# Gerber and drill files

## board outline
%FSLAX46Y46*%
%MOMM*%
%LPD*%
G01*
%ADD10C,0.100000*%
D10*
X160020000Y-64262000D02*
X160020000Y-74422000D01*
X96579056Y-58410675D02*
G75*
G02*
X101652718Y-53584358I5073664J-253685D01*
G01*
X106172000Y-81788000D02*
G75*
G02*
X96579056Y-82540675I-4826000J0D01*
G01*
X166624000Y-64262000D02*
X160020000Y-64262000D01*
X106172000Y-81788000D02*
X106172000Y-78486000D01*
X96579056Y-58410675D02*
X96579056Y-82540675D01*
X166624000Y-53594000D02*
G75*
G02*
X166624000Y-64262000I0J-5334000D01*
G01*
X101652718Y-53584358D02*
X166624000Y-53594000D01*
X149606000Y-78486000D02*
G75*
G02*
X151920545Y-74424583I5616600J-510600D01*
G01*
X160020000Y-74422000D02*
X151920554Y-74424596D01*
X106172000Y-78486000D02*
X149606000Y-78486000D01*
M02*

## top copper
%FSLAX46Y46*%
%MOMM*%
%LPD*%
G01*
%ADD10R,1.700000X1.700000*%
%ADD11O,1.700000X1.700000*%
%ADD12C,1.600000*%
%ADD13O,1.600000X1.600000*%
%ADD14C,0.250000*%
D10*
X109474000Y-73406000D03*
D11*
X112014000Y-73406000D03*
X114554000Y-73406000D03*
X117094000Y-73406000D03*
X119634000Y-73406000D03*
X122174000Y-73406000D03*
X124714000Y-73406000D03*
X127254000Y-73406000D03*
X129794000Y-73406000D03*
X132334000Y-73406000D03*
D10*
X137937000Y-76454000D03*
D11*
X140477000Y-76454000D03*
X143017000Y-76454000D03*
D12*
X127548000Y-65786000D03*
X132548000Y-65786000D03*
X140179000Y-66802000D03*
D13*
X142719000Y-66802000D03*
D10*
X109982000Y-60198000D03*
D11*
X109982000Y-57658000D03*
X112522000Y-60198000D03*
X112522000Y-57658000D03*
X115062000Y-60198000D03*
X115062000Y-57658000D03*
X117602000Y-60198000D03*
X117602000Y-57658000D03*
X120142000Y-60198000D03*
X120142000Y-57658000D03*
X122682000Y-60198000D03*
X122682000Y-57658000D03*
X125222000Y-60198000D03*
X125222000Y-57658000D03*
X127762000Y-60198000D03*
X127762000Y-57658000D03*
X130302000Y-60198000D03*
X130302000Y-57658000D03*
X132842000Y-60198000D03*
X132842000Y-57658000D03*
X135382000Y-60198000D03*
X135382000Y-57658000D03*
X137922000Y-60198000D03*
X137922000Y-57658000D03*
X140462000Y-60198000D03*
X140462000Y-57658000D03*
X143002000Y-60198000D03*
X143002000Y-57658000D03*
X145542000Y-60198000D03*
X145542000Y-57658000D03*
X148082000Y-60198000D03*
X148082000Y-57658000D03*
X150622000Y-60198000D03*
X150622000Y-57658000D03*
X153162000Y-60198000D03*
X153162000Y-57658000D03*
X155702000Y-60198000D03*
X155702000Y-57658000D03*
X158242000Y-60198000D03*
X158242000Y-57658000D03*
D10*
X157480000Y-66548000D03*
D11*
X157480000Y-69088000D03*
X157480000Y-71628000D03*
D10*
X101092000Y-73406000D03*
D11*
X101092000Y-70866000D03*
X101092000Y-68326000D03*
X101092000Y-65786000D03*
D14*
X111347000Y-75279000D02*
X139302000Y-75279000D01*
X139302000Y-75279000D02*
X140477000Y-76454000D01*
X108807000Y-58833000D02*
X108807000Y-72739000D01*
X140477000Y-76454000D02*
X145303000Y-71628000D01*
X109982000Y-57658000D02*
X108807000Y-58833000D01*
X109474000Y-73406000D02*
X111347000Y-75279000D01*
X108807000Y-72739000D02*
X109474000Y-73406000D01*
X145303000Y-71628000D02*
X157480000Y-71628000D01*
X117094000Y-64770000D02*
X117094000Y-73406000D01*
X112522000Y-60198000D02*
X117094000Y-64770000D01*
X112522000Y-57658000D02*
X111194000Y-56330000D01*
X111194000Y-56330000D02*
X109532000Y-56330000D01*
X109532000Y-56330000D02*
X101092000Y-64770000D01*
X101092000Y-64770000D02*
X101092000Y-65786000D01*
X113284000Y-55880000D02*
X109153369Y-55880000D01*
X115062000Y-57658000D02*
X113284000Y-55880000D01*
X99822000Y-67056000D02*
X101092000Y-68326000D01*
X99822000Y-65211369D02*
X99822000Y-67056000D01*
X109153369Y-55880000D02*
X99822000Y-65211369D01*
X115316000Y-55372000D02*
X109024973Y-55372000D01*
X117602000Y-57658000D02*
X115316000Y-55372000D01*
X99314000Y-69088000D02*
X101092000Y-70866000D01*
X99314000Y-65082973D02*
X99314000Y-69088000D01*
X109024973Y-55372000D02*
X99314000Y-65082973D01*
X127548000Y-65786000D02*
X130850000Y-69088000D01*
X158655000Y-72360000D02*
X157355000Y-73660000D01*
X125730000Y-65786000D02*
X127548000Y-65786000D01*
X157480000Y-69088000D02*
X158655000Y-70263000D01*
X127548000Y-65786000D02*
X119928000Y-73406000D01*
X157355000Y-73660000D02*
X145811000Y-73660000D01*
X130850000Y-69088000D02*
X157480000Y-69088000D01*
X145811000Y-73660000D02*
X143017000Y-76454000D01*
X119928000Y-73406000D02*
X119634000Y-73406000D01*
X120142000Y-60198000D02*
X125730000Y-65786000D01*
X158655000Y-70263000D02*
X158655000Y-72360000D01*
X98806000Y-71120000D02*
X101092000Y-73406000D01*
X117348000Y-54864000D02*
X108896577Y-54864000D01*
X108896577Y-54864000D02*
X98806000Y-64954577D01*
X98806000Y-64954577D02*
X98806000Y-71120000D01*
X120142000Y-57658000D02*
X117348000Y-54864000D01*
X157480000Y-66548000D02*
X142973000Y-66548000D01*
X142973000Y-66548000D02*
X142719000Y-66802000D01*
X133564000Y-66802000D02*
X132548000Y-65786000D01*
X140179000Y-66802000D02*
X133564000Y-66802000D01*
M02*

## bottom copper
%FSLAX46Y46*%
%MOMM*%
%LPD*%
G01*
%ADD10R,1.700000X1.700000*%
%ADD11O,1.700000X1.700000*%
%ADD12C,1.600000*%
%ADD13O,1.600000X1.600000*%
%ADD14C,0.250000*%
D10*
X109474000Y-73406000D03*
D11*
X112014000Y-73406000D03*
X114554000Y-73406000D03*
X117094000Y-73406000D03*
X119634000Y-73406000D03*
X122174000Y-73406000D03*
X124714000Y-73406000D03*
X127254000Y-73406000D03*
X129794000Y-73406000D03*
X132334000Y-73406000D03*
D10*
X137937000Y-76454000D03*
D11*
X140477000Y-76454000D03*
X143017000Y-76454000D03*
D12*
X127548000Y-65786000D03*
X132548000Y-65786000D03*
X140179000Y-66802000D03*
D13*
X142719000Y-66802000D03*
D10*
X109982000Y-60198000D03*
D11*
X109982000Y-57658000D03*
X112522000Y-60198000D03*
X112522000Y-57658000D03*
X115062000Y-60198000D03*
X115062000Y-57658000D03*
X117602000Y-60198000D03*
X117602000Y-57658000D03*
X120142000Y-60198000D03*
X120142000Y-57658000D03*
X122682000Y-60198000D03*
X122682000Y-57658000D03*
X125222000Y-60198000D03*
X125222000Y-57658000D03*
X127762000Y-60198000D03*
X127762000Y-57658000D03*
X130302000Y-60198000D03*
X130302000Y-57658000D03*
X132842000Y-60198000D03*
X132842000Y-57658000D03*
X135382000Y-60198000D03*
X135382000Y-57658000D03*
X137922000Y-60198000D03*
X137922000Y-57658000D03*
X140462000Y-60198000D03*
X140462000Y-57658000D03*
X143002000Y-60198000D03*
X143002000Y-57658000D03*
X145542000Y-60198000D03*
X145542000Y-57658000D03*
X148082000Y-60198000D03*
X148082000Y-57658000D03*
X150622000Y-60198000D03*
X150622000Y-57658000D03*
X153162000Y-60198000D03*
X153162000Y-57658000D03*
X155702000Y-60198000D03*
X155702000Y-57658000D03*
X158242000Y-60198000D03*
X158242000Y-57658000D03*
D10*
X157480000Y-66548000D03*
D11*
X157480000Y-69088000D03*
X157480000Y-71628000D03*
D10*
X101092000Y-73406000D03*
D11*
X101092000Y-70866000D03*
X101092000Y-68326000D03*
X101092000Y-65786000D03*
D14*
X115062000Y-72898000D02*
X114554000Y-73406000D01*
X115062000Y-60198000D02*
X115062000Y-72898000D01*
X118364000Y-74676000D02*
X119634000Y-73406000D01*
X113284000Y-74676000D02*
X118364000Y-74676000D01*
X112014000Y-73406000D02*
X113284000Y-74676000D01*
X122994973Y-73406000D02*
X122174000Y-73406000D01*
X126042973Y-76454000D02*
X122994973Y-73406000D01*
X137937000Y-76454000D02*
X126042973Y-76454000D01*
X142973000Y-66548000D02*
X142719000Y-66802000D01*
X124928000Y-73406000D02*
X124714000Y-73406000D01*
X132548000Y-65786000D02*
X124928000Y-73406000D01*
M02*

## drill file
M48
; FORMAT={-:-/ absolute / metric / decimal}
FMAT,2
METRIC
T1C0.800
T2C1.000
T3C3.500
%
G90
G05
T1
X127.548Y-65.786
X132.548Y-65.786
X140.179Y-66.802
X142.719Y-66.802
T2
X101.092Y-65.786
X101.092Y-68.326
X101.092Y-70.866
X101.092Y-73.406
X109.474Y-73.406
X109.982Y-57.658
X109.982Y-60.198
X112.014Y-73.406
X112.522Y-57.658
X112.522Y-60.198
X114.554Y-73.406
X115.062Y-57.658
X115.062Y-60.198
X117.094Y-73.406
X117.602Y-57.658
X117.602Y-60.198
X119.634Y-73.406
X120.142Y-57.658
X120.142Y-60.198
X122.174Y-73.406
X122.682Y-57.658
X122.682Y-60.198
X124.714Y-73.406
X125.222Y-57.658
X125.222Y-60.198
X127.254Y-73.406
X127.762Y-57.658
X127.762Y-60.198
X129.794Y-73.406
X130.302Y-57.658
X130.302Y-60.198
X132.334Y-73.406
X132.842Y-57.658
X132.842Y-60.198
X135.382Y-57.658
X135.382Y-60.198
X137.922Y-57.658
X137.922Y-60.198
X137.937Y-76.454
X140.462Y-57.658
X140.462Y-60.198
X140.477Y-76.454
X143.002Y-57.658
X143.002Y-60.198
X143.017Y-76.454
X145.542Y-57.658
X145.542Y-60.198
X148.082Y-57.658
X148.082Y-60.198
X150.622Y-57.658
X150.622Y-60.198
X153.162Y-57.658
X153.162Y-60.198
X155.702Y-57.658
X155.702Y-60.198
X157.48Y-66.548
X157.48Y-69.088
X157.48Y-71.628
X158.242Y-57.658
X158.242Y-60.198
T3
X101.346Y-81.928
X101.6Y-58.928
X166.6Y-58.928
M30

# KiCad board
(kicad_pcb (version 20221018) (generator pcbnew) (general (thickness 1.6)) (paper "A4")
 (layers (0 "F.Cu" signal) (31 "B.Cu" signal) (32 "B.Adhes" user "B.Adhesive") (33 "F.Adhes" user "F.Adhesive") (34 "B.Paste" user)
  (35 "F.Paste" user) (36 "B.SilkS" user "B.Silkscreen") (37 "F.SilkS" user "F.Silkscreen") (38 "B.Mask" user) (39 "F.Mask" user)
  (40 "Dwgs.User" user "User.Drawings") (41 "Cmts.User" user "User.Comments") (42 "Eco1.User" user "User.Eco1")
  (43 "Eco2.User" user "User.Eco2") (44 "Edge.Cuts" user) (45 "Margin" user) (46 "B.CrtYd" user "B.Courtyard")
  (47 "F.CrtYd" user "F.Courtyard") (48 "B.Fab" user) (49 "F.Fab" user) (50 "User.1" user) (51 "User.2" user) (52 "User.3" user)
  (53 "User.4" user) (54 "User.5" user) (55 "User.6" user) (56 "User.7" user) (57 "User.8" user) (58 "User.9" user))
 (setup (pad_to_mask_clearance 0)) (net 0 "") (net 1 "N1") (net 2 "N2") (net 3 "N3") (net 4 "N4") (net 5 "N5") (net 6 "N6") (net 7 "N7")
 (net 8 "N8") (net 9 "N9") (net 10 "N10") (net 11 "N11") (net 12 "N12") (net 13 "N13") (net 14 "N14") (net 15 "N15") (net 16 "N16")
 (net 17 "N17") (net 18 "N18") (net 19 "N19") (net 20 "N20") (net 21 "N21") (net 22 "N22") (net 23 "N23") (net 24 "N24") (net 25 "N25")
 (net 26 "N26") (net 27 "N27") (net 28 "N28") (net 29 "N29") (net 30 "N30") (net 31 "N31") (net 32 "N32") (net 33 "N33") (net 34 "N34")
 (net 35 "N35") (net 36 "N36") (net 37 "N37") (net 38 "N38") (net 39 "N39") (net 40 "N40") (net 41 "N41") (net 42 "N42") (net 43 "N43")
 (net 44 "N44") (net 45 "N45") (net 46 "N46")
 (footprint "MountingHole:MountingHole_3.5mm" (layer "F.Cu") (at 166.6 58.928)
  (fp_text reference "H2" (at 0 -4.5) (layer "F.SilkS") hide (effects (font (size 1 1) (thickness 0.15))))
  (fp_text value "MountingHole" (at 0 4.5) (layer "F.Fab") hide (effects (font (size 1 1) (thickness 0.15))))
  (pad "" np_thru_hole circle (at 0 0) (size 3.5 3.5) (drill 3.5) (layers "*.Cu" "*.Mask")))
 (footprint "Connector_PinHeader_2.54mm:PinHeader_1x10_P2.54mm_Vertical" (layer "F.Cu") (at 109.474 73.406 90)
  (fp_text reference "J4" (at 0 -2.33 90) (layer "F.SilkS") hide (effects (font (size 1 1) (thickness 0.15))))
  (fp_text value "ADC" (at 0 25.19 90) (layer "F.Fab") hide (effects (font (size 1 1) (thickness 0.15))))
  (pad "1" thru_hole rect (at 0 0 90) (size 1.7 1.7) (drill 1) (layers "*.Cu" "*.Mask") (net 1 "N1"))
  (pad "2" thru_hole oval (at 0 2.54 90) (size 1.7 1.7) (drill 1) (layers "*.Cu" "*.Mask") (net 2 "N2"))
  (pad "3" thru_hole oval (at 0 5.08 90) (size 1.7 1.7) (drill 1) (layers "*.Cu" "*.Mask") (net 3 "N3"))
  (pad "4" thru_hole oval (at 0 7.62 90) (size 1.7 1.7) (drill 1) (layers "*.Cu" "*.Mask") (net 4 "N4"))
  (pad "5" thru_hole oval (at 0 10.16 90) (size 1.7 1.7) (drill 1) (layers "*.Cu" "*.Mask") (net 2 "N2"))
  (pad "6" thru_hole oval (at 0 12.7 90) (size 1.7 1.7) (drill 1) (layers "*.Cu" "*.Mask") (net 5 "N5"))
  (pad "7" thru_hole oval (at 0 15.24 90) (size 1.7 1.7) (drill 1) (layers "*.Cu" "*.Mask") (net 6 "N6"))
  (pad "8" thru_hole oval (at 0 17.78 90) (size 1.7 1.7) (drill 1) (layers "*.Cu" "*.Mask") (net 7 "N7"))
  (pad "9" thru_hole oval (at 0 20.32 90) (size 1.7 1.7) (drill 1) (layers "*.Cu" "*.Mask") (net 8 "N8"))
  (pad "10" thru_hole oval (at 0 22.86 90) (size 1.7 1.7) (drill 1) (layers "*.Cu" "*.Mask") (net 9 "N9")))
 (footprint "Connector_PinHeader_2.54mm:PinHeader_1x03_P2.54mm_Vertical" (layer "F.Cu") (at 137.937 76.454 90)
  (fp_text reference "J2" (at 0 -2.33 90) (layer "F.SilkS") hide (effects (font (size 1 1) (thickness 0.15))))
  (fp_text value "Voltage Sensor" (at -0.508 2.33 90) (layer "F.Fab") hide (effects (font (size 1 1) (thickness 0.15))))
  (pad "1" thru_hole rect (at 0 0 90) (size 1.7 1.7) (drill 1) (layers "*.Cu" "*.Mask") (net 5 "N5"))
  (pad "2" thru_hole oval (at 0 2.54 90) (size 1.7 1.7) (drill 1) (layers "*.Cu" "*.Mask") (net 1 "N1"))
  (pad "3" thru_hole oval (at 0 5.08 90) (size 1.7 1.7) (drill 1) (layers "*.Cu" "*.Mask") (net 2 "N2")))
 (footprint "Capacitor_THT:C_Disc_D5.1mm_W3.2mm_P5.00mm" (layer "F.Cu") (at 127.548 65.786)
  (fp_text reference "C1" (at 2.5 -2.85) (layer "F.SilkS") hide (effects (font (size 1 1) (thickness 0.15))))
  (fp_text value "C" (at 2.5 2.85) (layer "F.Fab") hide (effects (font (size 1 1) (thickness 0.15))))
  (pad "1" thru_hole circle (at 0 0) (size 1.6 1.6) (drill 0.8) (layers "*.Cu" "*.Mask") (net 2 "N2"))
  (pad "2" thru_hole circle (at 5 0) (size 1.6 1.6) (drill 0.8) (layers "*.Cu" "*.Mask") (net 6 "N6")))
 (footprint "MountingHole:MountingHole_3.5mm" (layer "F.Cu") (at 101.346 81.928)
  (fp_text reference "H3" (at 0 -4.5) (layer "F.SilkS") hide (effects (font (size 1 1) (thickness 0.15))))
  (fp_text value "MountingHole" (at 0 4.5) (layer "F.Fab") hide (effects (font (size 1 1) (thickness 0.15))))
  (pad "" np_thru_hole circle (at 0 0) (size 3.5 3.5) (drill 3.5) (layers "*.Cu" "*.Mask")))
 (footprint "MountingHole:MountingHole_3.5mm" (layer "F.Cu") (at 101.6 58.928)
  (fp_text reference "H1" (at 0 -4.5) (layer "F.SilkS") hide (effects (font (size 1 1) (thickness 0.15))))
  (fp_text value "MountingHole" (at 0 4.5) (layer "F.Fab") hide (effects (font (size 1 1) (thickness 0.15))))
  (pad "" np_thru_hole circle (at 0 0) (size 3.5 3.5) (drill 3.5) (layers "*.Cu" "*.Mask")))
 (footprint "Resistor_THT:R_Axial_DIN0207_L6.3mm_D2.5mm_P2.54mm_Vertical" (layer "F.Cu") (at 140.179 66.802)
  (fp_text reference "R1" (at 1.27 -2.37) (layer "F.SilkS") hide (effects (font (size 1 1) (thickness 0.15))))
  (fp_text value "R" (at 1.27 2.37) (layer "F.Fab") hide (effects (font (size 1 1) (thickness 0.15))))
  (pad "1" thru_hole circle (at 0 0) (size 1.6 1.6) (drill 0.8) (layers "*.Cu" "*.Mask") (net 6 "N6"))
  (pad "2" thru_hole oval (at 2.54 0) (size 1.6 1.6) (drill 0.8) (layers "*.Cu" "*.Mask") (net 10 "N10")))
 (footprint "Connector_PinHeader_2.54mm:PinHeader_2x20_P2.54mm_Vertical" (layer "F.Cu") (at 109.982 60.198 90)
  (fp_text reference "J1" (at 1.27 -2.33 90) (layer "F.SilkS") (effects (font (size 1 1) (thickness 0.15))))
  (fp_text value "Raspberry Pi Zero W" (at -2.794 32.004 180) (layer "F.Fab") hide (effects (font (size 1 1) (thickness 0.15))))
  (pad "1" thru_hole rect (at 0 0 90) (size 1.7 1.7) (drill 1) (layers "*.Cu" "*.Mask") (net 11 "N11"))
  (pad "2" thru_hole oval (at 2.54 0 90) (size 1.7 1.7) (drill 1) (layers "*.Cu" "*.Mask") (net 1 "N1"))
  (pad "3" thru_hole oval (at 0 2.54 90) (size 1.7 1.7) (drill 1) (layers "*.Cu" "*.Mask") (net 4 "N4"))
  (pad "4" thru_hole oval (at 2.54 2.54 90) (size 1.7 1.7) (drill 1) (layers "*.Cu" "*.Mask") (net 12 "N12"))
  (pad "5" thru_hole oval (at 0 5.08 90) (size 1.7 1.7) (drill 1) (layers "*.Cu" "*.Mask") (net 3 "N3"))
  (pad "6" thru_hole oval (at 2.54 5.08 90) (size 1.7 1.7) (drill 1) (layers "*.Cu" "*.Mask") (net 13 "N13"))
  (pad "7" thru_hole oval (at 0 7.62 90) (size 1.7 1.7) (drill 1) (layers "*.Cu" "*.Mask") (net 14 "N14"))
  (pad "8" thru_hole oval (at 2.54 7.62 90) (size 1.7 1.7) (drill 1) (layers "*.Cu" "*.Mask") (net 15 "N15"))
  (pad "9" thru_hole oval (at 0 10.16 90) (size 1.7 1.7) (drill 1) (layers "*.Cu" "*.Mask") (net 2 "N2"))
  (pad "10" thru_hole oval (at 2.54 10.16 90) (size 1.7 1.7) (drill 1) (layers "*.Cu" "*.Mask") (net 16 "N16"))
  (pad "11" thru_hole oval (at 0 12.7 90) (size 1.7 1.7) (drill 1) (layers "*.Cu" "*.Mask") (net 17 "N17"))
  (pad "12" thru_hole oval (at 2.54 12.7 90) (size 1.7 1.7) (drill 1) (layers "*.Cu" "*.Mask") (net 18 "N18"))
  (pad "13" thru_hole oval (at 0 15.24 90) (size 1.7 1.7) (drill 1) (layers "*.Cu" "*.Mask") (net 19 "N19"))
  (pad "14" thru_hole oval (at 2.54 15.24 90) (size 1.7 1.7) (drill 1) (layers "*.Cu" "*.Mask") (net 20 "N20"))
  (pad "15" thru_hole oval (at 0 17.78 90) (size 1.7 1.7) (drill 1) (layers "*.Cu" "*.Mask") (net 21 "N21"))
  (pad "16" thru_hole oval (at 2.54 17.78 90) (size 1.7 1.7) (drill 1) (layers "*.Cu" "*.Mask") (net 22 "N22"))
  (pad "17" thru_hole oval (at 0 20.32 90) (size 1.7 1.7) (drill 1) (layers "*.Cu" "*.Mask") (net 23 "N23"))
  (pad "18" thru_hole oval (at 2.54 20.32 90) (size 1.7 1.7) (drill 1) (layers "*.Cu" "*.Mask") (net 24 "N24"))
  (pad "19" thru_hole oval (at 0 22.86 90) (size 1.7 1.7) (drill 1) (layers "*.Cu" "*.Mask") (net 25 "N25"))
  (pad "20" thru_hole oval (at 2.54 22.86 90) (size 1.7 1.7) (drill 1) (layers "*.Cu" "*.Mask") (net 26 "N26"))
  (pad "21" thru_hole oval (at 0 25.4 90) (size 1.7 1.7) (drill 1) (layers "*.Cu" "*.Mask") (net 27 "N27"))
  (pad "22" thru_hole oval (at 2.54 25.4 90) (size 1.7 1.7) (drill 1) (layers "*.Cu" "*.Mask") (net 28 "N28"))
  (pad "23" thru_hole oval (at 0 27.94 90) (size 1.7 1.7) (drill 1) (layers "*.Cu" "*.Mask") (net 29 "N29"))
  (pad "24" thru_hole oval (at 2.54 27.94 90) (size 1.7 1.7) (drill 1) (layers "*.Cu" "*.Mask") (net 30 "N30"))
  (pad "25" thru_hole oval (at 0 30.48 90) (size 1.7 1.7) (drill 1) (layers "*.Cu" "*.Mask") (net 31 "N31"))
  (pad "26" thru_hole oval (at 2.54 30.48 90) (size 1.7 1.7) (drill 1) (layers "*.Cu" "*.Mask") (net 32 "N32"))
  (pad "27" thru_hole oval (at 0 33.02 90) (size 1.7 1.7) (drill 1) (layers "*.Cu" "*.Mask") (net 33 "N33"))
  (pad "28" thru_hole oval (at 2.54 33.02 90) (size 1.7 1.7) (drill 1) (layers "*.Cu" "*.Mask") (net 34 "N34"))
  (pad "29" thru_hole oval (at 0 35.56 90) (size 1.7 1.7) (drill 1) (layers "*.Cu" "*.Mask") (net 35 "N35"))
  (pad "30" thru_hole oval (at 2.54 35.56 90) (size 1.7 1.7) (drill 1) (layers "*.Cu" "*.Mask") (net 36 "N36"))
  (pad "31" thru_hole oval (at 0 38.1 90) (size 1.7 1.7) (drill 1) (layers "*.Cu" "*.Mask") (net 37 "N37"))
  (pad "32" thru_hole oval (at 2.54 38.1 90) (size 1.7 1.7) (drill 1) (layers "*.Cu" "*.Mask") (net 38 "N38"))
  (pad "33" thru_hole oval (at 0 40.64 90) (size 1.7 1.7) (drill 1) (layers "*.Cu" "*.Mask") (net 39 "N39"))
  (pad "34" thru_hole oval (at 2.54 40.64 90) (size 1.7 1.7) (drill 1) (layers "*.Cu" "*.Mask") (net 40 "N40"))
  (pad "35" thru_hole oval (at 0 43.18 90) (size 1.7 1.7) (drill 1) (layers "*.Cu" "*.Mask") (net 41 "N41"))
  (pad "36" thru_hole oval (at 2.54 43.18 90) (size 1.7 1.7) (drill 1) (layers "*.Cu" "*.Mask") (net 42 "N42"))
  (pad "37" thru_hole oval (at 0 45.72 90) (size 1.7 1.7) (drill 1) (layers "*.Cu" "*.Mask") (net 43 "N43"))
  (pad "38" thru_hole oval (at 2.54 45.72 90) (size 1.7 1.7) (drill 1) (layers "*.Cu" "*.Mask") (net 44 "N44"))
  (pad "39" thru_hole oval (at 0 48.26 90) (size 1.7 1.7) (drill 1) (layers "*.Cu" "*.Mask") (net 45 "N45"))
  (pad "40" thru_hole oval (at 2.54 48.26 90) (size 1.7 1.7) (drill 1) (layers "*.Cu" "*.Mask") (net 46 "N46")))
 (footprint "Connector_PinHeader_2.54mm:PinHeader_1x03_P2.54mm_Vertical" (layer "F.Cu") (at 157.48 66.548)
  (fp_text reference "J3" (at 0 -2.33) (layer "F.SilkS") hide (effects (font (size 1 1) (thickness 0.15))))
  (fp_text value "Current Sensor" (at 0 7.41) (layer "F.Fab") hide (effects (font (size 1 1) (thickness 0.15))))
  (pad "1" thru_hole rect (at 0 0) (size 1.7 1.7) (drill 1) (layers "*.Cu" "*.Mask") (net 10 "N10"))
  (pad "2" thru_hole oval (at 0 2.54) (size 1.7 1.7) (drill 1) (layers "*.Cu" "*.Mask") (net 2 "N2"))
  (pad "3" thru_hole oval (at 0 5.08) (size 1.7 1.7) (drill 1) (layers "*.Cu" "*.Mask") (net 1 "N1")))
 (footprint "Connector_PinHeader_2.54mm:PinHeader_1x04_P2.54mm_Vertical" (layer "F.Cu") (at 101.092 73.406 180)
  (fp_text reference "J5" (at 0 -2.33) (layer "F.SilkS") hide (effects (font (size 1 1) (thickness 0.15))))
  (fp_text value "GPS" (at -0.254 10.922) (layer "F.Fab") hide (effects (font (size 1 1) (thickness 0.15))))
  (pad "1" thru_hole rect (at 0 0 180) (size 1.7 1.7) (drill 1) (layers "*.Cu" "*.Mask") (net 16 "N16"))
  (pad "2" thru_hole oval (at 0 2.54 180) (size 1.7 1.7) (drill 1) (layers "*.Cu" "*.Mask") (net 15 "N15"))
  (pad "3" thru_hole oval (at 0 5.08 180) (size 1.7 1.7) (drill 1) (layers "*.Cu" "*.Mask") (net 13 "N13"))
  (pad "4" thru_hole oval (at 0 7.62 180) (size 1.7 1.7) (drill 1) (layers "*.Cu" "*.Mask") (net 12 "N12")))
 (gr_line (start 160.02 64.262) (end 160.02 74.422) (stroke (width 0.1) (type default)) (layer "Edge.Cuts"))
 (gr_arc (start 96.579056 58.410675) (mid 98.151455 54.983658) (end 101.652718 53.584358) (stroke (width 0.1) (type default))
  (layer "Edge.Cuts"))
 (gr_arc (start 106.172 81.788) (mid 101.723494 86.599213) (end 96.579056 82.540675) (stroke (width 0.1) (type default)) (layer "Edge.Cuts"))
 (gr_line (start 166.624 64.262) (end 160.02 64.262) (stroke (width 0.1) (type default)) (layer "Edge.Cuts"))
 (gr_line (start 106.172 81.788) (end 106.172 78.486) (stroke (width 0.1) (type default)) (layer "Edge.Cuts"))
 (gr_line (start 96.579056 58.410675) (end 96.579056 82.540675) (stroke (width 0.1) (type default)) (layer "Edge.Cuts"))
 (gr_arc (start 166.624 53.594) (mid 171.958 58.928) (end 166.624 64.262) (stroke (width 0.1) (type default)) (layer "Edge.Cuts"))
 (gr_line (start 101.652718 53.584358) (end 166.624 53.594) (stroke (width 0.1) (type default)) (layer "Edge.Cuts"))
 (gr_arc (start 149.606 78.486) (mid 150.322666 76.204198) (end 151.920554 74.424596) (stroke (width 0.1) (type default))
  (layer "Edge.Cuts"))
 (gr_line (start 160.02 74.422) (end 151.920554 74.424596) (stroke (width 0.1) (type default)) (layer "Edge.Cuts"))
 (gr_line (start 106.172 78.486) (end 149.606 78.486) (stroke (width 0.1) (type default)) (layer "Edge.Cuts"))
 (segment (start 111.347 75.279) (end 139.302 75.279) (width 0.25) (layer "F.Cu") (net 1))
 (segment (start 139.302 75.279) (end 140.477 76.454) (width 0.25) (layer "F.Cu") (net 1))
 (segment (start 108.807 58.833) (end 108.807 72.739) (width 0.25) (layer "F.Cu") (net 1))
 (segment (start 140.477 76.454) (end 145.303 71.628) (width 0.25) (layer "F.Cu") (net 1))
 (segment (start 109.982 57.658) (end 108.807 58.833) (width 0.25) (layer "F.Cu") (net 1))
 (segment (start 109.474 73.406) (end 111.347 75.279) (width 0.25) (layer "F.Cu") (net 1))
 (segment (start 108.807 72.739) (end 109.474 73.406) (width 0.25) (layer "F.Cu") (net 1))
 (segment (start 145.303 71.628) (end 157.48 71.628) (width 0.25) (layer "F.Cu") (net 1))
 (segment (start 117.094 64.77) (end 117.094 73.406) (width 0.25) (layer "F.Cu") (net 4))
 (segment (start 112.522 60.198) (end 117.094 64.77) (width 0.25) (layer "F.Cu") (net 4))
 (segment (start 112.522 57.658) (end 111.194 56.33) (width 0.25) (layer "F.Cu") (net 12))
 (segment (start 111.194 56.33) (end 109.532 56.33) (width 0.25) (layer "F.Cu") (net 12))
 (segment (start 109.532 56.33) (end 101.092 64.77) (width 0.25) (layer "F.Cu") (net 12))
 (segment (start 101.092 64.77) (end 101.092 65.786) (width 0.25) (layer "F.Cu") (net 12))
 (segment (start 115.062 72.898) (end 114.554 73.406) (width 0.25) (layer "B.Cu") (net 3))
 (segment (start 115.062 60.198) (end 115.062 72.898) (width 0.25) (layer "B.Cu") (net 3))
 (segment (start 113.284 55.88) (end 109.153369 55.88) (width 0.25) (layer "F.Cu") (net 13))
 (segment (start 115.062 57.658) (end 113.284 55.88) (width 0.25) (layer "F.Cu") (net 13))
 (segment (start 99.822 67.056) (end 101.092 68.326) (width 0.25) (layer "F.Cu") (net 13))
 (segment (start 99.822 65.211369) (end 99.822 67.056) (width 0.25) (layer "F.Cu") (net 13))
 (segment (start 109.153369 55.88) (end 99.822 65.211369) (width 0.25) (layer "F.Cu") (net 13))
 (segment (start 115.316 55.372) (end 109.024973 55.372) (width 0.25) (layer "F.Cu") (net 15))
 (segment (start 117.602 57.658) (end 115.316 55.372) (width 0.25) (layer "F.Cu") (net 15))
 (segment (start 99.314 69.088) (end 101.092 70.866) (width 0.25) (layer "F.Cu") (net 15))
 (segment (start 99.314 65.082973) (end 99.314 69.088) (width 0.25) (layer "F.Cu") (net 15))
 (segment (start 109.024973 55.372) (end 99.314 65.082973) (width 0.25) (layer "F.Cu") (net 15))
 (segment (start 127.548 65.786) (end 130.85 69.088) (width 0.25) (layer "F.Cu") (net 2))
 (segment (start 158.655 72.36) (end 157.355 73.66) (width 0.25) (layer "F.Cu") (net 2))
 (segment (start 125.73 65.786) (end 127.548 65.786) (width 0.25) (layer "F.Cu") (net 2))
 (segment (start 157.48 69.088) (end 158.655 70.263) (width 0.25) (layer "F.Cu") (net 2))
 (segment (start 127.548 65.786) (end 119.928 73.406) (width 0.25) (layer "F.Cu") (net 2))
 (segment (start 157.355 73.66) (end 145.811 73.66) (width 0.25) (layer "F.Cu") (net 2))
 (segment (start 130.85 69.088) (end 157.48 69.088) (width 0.25) (layer "F.Cu") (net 2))
 (segment (start 145.811 73.66) (end 143.017 76.454) (width 0.25) (layer "F.Cu") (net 2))
 (segment (start 119.928 73.406) (end 119.634 73.406) (width 0.25) (layer "F.Cu") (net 2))
 (segment (start 120.142 60.198) (end 125.73 65.786) (width 0.25) (layer "F.Cu") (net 2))
 (segment (start 158.655 70.263) (end 158.655 72.36) (width 0.25) (layer "F.Cu") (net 2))
 (segment (start 118.364 74.676) (end 119.634 73.406) (width 0.25) (layer "B.Cu") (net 2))
 (segment (start 113.284 74.676) (end 118.364 74.676) (width 0.25) (layer "B.Cu") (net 2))
 (segment (start 112.014 73.406) (end 113.284 74.676) (width 0.25) (layer "B.Cu") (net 2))
 (segment (start 98.806 71.12) (end 101.092 73.406) (width 0.25) (layer "F.Cu") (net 16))
 (segment (start 117.348 54.864) (end 108.896577 54.864) (width 0.25) (layer "F.Cu") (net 16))
 (segment (start 108.896577 54.864) (end 98.806 64.954577) (width 0.25) (layer "F.Cu") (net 16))
 (segment (start 98.806 64.954577) (end 98.806 71.12) (width 0.25) (layer "F.Cu") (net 16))
 (segment (start 120.142 57.658) (end 117.348 54.864) (width 0.25) (layer "F.Cu") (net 16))
 (segment (start 122.994973 73.406) (end 122.174 73.406) (width 0.25) (layer "B.Cu") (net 5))
 (segment (start 126.042973 76.454) (end 122.994973 73.406) (width 0.25) (layer "B.Cu") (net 5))
 (segment (start 137.937 76.454) (end 126.042973 76.454) (width 0.25) (layer "B.Cu") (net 5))
 (segment (start 157.48 66.548) (end 142.973 66.548) (width 0.25) (layer "F.Cu") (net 10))
 (segment (start 142.973 66.548) (end 142.719 66.802) (width 0.25) (layer "F.Cu") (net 10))
 (segment (start 142.973 66.548) (end 142.719 66.802) (width 0.25) (layer "B.Cu") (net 10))
 (segment (start 133.564 66.802) (end 132.548 65.786) (width 0.25) (layer "F.Cu") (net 6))
 (segment (start 140.179 66.802) (end 133.564 66.802) (width 0.25) (layer "F.Cu") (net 6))
 (segment (start 124.928 73.406) (end 124.714 73.406) (width 0.25) (layer "B.Cu") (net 6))
 (segment (start 132.548 65.786) (end 124.928 73.406) (width 0.25) (layer "B.Cu") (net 6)))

